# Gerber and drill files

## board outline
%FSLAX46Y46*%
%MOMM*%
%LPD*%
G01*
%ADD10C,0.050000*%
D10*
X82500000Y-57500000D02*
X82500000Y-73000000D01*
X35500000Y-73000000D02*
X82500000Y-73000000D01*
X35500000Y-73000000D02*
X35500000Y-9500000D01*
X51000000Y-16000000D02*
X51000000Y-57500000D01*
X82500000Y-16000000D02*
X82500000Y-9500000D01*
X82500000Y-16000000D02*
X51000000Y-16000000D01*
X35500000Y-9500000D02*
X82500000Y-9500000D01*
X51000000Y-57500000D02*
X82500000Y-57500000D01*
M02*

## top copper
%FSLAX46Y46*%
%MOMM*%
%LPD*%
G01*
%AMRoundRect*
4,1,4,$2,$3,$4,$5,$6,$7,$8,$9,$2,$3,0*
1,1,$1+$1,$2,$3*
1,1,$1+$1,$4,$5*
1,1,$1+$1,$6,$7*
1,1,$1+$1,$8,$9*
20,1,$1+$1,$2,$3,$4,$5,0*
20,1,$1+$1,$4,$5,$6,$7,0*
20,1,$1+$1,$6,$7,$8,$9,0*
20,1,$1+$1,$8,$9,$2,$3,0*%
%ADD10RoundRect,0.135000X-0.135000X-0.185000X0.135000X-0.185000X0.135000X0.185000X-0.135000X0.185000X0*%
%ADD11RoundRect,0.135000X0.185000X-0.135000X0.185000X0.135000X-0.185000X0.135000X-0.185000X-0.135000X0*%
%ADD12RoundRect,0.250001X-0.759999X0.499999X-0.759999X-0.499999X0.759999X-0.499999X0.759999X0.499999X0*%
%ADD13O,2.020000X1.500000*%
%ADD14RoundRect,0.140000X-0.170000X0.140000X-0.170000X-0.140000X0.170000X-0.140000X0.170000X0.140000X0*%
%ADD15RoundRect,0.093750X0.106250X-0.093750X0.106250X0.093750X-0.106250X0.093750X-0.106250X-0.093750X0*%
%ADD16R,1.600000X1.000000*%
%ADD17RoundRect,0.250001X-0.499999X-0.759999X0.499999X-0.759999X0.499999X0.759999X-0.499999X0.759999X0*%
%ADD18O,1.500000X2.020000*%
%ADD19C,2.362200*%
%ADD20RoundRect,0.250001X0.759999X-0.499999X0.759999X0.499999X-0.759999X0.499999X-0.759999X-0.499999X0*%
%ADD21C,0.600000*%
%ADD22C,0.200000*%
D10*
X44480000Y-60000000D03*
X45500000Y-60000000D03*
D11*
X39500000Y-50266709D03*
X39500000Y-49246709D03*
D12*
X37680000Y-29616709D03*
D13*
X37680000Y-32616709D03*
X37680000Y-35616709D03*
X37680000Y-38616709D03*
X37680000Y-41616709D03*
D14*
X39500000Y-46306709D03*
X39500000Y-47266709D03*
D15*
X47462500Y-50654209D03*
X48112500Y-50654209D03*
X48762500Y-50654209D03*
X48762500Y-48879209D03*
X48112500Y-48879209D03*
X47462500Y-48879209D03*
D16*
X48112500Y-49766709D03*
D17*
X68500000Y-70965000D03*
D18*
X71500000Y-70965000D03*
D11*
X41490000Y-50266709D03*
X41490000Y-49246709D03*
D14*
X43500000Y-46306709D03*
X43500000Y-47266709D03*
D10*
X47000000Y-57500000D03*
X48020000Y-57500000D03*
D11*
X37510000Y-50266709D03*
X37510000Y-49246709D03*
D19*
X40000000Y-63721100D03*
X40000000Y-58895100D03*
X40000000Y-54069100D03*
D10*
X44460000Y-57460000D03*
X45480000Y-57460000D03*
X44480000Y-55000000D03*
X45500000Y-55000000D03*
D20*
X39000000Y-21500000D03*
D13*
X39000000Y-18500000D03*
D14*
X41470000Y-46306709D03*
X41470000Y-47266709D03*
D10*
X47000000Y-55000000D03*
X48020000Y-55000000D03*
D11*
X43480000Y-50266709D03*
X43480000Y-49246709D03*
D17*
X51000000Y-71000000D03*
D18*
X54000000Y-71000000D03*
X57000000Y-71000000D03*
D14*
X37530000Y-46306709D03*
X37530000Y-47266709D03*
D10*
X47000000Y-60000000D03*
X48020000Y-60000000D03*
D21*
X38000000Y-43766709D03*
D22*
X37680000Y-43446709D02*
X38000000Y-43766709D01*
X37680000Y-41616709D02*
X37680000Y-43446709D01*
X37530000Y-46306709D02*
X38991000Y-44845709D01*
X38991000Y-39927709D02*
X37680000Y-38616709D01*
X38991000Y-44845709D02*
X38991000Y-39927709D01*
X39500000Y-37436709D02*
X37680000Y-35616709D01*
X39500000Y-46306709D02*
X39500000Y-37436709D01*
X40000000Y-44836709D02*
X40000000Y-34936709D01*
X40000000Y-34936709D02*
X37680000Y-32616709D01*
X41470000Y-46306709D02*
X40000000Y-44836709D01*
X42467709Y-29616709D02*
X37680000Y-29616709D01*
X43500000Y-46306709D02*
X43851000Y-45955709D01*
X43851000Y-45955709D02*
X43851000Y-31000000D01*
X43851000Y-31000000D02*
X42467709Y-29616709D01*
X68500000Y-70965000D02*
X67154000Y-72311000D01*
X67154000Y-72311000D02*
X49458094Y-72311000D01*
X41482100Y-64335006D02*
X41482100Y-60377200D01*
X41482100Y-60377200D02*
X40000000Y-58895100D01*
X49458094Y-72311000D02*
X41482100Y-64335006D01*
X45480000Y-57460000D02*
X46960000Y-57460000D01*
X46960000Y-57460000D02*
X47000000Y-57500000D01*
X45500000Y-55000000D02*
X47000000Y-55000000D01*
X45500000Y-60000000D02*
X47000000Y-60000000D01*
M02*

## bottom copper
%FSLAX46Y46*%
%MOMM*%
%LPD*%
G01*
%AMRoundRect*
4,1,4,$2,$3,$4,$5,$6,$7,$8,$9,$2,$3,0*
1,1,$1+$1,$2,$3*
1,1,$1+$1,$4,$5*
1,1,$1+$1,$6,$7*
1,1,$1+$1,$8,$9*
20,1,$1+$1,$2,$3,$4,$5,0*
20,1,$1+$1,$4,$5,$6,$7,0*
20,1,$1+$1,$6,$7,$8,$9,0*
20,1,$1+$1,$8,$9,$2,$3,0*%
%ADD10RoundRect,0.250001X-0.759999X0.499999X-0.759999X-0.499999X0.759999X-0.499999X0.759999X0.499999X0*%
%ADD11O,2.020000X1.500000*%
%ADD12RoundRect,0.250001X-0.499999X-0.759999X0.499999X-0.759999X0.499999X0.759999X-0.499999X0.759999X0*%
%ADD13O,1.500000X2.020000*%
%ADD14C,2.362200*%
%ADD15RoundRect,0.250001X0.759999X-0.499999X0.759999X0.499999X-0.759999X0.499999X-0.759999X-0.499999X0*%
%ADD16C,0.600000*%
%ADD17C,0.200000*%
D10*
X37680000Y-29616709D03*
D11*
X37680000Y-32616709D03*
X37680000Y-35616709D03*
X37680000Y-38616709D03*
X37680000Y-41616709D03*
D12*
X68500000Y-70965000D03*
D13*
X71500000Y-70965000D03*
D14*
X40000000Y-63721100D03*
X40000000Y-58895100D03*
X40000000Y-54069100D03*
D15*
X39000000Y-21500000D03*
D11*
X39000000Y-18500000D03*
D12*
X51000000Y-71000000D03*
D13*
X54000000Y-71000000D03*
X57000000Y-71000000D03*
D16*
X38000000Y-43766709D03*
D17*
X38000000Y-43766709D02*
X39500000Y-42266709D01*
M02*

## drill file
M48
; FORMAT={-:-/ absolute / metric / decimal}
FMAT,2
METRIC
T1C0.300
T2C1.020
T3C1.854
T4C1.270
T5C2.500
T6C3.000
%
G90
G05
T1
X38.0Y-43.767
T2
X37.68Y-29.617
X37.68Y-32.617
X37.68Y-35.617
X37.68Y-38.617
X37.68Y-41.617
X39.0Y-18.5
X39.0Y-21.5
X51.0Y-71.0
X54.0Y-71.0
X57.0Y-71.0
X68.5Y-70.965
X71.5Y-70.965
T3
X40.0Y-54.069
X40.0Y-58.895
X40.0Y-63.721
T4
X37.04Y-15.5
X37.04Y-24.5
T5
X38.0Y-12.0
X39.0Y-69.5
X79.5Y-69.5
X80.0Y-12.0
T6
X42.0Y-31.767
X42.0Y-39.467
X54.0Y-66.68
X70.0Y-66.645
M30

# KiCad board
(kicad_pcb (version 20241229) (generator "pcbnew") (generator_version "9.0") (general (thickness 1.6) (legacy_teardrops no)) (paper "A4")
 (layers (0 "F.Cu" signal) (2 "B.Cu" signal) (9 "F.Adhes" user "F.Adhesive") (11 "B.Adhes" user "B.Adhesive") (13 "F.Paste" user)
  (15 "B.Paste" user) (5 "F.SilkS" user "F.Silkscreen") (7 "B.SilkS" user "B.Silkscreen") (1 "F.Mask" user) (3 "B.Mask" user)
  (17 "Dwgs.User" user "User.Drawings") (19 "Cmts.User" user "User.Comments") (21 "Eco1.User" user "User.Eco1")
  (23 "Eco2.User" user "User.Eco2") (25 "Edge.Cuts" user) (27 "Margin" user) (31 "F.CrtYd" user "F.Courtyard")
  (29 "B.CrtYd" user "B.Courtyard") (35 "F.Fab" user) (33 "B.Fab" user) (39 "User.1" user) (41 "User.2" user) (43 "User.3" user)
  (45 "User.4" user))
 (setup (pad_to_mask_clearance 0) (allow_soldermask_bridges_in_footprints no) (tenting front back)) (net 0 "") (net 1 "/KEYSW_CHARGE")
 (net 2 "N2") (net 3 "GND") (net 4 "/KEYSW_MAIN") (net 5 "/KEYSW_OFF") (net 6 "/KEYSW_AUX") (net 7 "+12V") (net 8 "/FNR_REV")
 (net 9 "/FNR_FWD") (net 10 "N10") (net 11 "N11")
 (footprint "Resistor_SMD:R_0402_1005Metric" (layer "F.Cu") (at 44.99 60)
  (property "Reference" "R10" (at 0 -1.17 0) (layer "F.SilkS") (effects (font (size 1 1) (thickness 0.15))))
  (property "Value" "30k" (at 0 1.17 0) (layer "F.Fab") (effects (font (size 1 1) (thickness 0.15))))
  (pad "1" smd roundrect (at -0.51 0) (size 0.54 0.64) (layers "F.Cu" "F.Mask" "F.Paste") (roundrect_rratio 0.25) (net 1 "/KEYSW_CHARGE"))
  (pad "2" smd roundrect (at 0.51 0) (size 0.54 0.64) (layers "F.Cu" "F.Mask" "F.Paste") (roundrect_rratio 0.25) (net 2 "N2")))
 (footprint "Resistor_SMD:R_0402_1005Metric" (layer "F.Cu") (at 39.5 49.756709 90)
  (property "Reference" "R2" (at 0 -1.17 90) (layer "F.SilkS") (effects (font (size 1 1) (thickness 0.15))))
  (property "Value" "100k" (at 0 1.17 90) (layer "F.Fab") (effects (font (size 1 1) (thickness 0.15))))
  (pad "1" smd roundrect (at -0.51 0 90) (size 0.54 0.64) (layers "F.Cu" "F.Mask" "F.Paste") (roundrect_rratio 0.25) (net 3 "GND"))
  (pad "2" smd roundrect (at 0.51 0 90) (size 0.54 0.64) (layers "F.Cu" "F.Mask" "F.Paste") (roundrect_rratio 0.25) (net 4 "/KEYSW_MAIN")))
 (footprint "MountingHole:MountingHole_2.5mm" (layer "F.Cu") (at 79.5 69.5)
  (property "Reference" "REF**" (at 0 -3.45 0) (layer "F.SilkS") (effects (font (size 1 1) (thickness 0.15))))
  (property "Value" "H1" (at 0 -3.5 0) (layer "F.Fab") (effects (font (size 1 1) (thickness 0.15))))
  (pad "" np_thru_hole circle (at 0 0) (size 2.5 2.5) (drill 2.5) (layers "*.Cu" "*.Mask")))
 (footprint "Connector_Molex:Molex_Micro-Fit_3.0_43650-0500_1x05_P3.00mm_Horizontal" (layer "F.Cu") (at 37.68 29.616709 -90)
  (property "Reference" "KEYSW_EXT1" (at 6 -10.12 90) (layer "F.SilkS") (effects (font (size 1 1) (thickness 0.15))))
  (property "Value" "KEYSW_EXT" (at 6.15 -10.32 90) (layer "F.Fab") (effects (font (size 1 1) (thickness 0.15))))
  (pad "" np_thru_hole circle (at 2.15 -4.32 270) (size 3 3) (drill 3) (layers "*.Cu" "*.Mask"))
  (pad "" np_thru_hole circle (at 9.85 -4.32 270) (size 3 3) (drill 3) (layers "*.Cu" "*.Mask"))
  (pad "1" thru_hole roundrect (at 0 0 270) (size 1.5 2.02) (drill 1.02) (layers "*.Cu" "*.Mask") (remove_unused_layers no)
   (roundrect_rratio 0.166667) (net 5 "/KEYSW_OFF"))
  (pad "2" thru_hole oval (at 3 0 270) (size 1.5 2.02) (drill 1.02) (layers "*.Cu" "*.Mask") (remove_unused_layers no) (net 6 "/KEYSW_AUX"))
  (pad "3" thru_hole oval (at 6 0 270) (size 1.5 2.02) (drill 1.02) (layers "*.Cu" "*.Mask") (remove_unused_layers no) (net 4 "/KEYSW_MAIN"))
  (pad "4" thru_hole oval (at 9 0 270) (size 1.5 2.02) (drill 1.02) (layers "*.Cu" "*.Mask") (remove_unused_layers no)
   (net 1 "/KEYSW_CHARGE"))
  (pad "5" thru_hole oval (at 12 0 270) (size 1.5 2.02) (drill 1.02) (layers "*.Cu" "*.Mask") (remove_unused_layers no) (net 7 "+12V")))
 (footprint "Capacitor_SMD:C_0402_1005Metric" (layer "F.Cu") (at 39.5 46.786709 -90)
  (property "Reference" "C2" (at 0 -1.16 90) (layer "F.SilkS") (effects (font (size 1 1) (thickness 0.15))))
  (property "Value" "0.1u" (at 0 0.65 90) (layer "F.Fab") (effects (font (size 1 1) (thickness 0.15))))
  (pad "1" smd roundrect (at -0.48 0 270) (size 0.56 0.62) (layers "F.Cu" "F.Mask" "F.Paste") (roundrect_rratio 0.25) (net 4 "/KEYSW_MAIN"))
  (pad "2" smd roundrect (at 0.48 0 270) (size 0.56 0.62) (layers "F.Cu" "F.Mask" "F.Paste") (roundrect_rratio 0.25) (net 3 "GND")))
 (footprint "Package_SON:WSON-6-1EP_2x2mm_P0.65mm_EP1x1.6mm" (layer "F.Cu") (at 48.1125 49.766709 90)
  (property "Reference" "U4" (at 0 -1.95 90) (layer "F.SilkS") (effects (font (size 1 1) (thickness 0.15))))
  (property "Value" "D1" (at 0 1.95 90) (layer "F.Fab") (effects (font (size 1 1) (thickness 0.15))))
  (pad "" smd roundrect (at 0 -0.4 90) (size 0.81 0.64) (layers "F.Paste") (roundrect_rratio 0.25))
  (pad "" smd roundrect (at 0 0.4 90) (size 0.81 0.64) (layers "F.Paste") (roundrect_rratio 0.25))
  (pad "1" smd roundrect (at -0.8875 -0.65 90) (size 0.375 0.4) (layers "F.Cu" "F.Mask" "F.Paste") (roundrect_rratio 0.25) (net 2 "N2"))
  (pad "2" smd roundrect (at -0.8875 0 90) (size 0.375 0.4) (layers "F.Cu" "F.Mask" "F.Paste") (roundrect_rratio 0.25) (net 2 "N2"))
  (pad "3" smd roundrect (at -0.8875 0.65 90) (size 0.375 0.4) (layers "F.Cu" "F.Mask" "F.Paste") (roundrect_rratio 0.25) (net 2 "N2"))
  (pad "4" smd roundrect (at 0.8875 0.65 90) (size 0.375 0.4) (layers "F.Cu" "F.Mask" "F.Paste") (roundrect_rratio 0.25) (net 3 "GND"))
  (pad "5" smd roundrect (at 0.8875 0 90) (size 0.375 0.4) (layers "F.Cu" "F.Mask" "F.Paste") (roundrect_rratio 0.25) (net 3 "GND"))
  (pad "6" smd roundrect (at 0.8875 -0.65 90) (size 0.375 0.4) (layers "F.Cu" "F.Mask" "F.Paste") (roundrect_rratio 0.25) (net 3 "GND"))
  (pad "7" smd rect (at 0 0 90) (size 1 1.6) (layers "F.Cu" "F.Mask") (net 2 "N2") (zone_connect 2)))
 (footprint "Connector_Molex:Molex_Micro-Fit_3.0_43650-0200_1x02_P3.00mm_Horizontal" (layer "F.Cu") (at 68.5 70.965)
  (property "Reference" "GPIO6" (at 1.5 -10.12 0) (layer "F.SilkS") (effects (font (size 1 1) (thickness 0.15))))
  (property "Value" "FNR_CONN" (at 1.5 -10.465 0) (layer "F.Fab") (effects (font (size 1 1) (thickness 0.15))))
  (pad "" np_thru_hole circle (at 1.5 -4.32) (size 3 3) (drill 3) (layers "*.Cu" "*.Mask"))
  (pad "1" thru_hole roundrect (at 0 0) (size 1.5 2.02) (drill 1.02) (layers "*.Cu" "*.Mask") (remove_unused_layers no)
   (roundrect_rratio 0.166667) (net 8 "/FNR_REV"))
  (pad "2" thru_hole oval (at 3 0) (size 1.5 2.02) (drill 1.02) (layers "*.Cu" "*.Mask") (remove_unused_layers no) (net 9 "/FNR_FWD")))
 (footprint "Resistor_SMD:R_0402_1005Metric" (layer "F.Cu") (at 41.49 49.756709 90)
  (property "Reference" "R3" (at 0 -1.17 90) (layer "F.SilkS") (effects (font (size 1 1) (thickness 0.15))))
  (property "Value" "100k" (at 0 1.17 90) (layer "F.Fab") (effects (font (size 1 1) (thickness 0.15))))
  (pad "1" smd roundrect (at -0.51 0 90) (size 0.54 0.64) (layers "F.Cu" "F.Mask" "F.Paste") (roundrect_rratio 0.25) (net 3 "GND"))
  (pad "2" smd roundrect (at 0.51 0 90) (size 0.54 0.64) (layers "F.Cu" "F.Mask" "F.Paste") (roundrect_rratio 0.25) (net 6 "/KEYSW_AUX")))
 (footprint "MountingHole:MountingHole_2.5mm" (layer "F.Cu") (at 39 69.5)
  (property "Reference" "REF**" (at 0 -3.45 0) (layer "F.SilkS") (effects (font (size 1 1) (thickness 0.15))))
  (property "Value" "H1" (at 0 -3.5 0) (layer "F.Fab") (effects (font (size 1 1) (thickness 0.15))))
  (pad "" np_thru_hole circle (at 0 0) (size 2.5 2.5) (drill 2.5) (layers "*.Cu" "*.Mask")))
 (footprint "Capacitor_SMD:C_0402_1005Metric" (layer "F.Cu") (at 43.5 46.786709 -90)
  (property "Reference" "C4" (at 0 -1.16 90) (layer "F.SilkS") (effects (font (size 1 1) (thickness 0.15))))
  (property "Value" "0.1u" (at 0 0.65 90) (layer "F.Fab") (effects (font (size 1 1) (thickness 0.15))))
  (pad "1" smd roundrect (at -0.48 0 270) (size 0.56 0.62) (layers "F.Cu" "F.Mask" "F.Paste") (roundrect_rratio 0.25) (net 5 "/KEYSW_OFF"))
  (pad "2" smd roundrect (at 0.48 0 270) (size 0.56 0.62) (layers "F.Cu" "F.Mask" "F.Paste") (roundrect_rratio 0.25) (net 3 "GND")))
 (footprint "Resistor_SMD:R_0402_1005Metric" (layer "F.Cu") (at 47.51 57.5)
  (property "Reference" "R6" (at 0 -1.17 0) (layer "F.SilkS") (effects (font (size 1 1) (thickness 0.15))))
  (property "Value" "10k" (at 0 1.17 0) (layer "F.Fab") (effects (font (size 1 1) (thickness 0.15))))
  (pad "1" smd roundrect (at -0.51 0) (size 0.54 0.64) (layers "F.Cu" "F.Mask" "F.Paste") (roundrect_rratio 0.25) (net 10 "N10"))
  (pad "2" smd roundrect (at 0.51 0) (size 0.54 0.64) (layers "F.Cu" "F.Mask" "F.Paste") (roundrect_rratio 0.25) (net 3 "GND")))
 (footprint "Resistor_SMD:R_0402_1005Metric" (layer "F.Cu") (at 37.51 49.756709 90)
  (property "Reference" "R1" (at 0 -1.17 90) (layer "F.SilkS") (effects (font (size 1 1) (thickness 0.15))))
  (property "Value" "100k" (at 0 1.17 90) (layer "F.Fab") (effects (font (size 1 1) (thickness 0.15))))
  (pad "1" smd roundrect (at -0.51 0 90) (size 0.54 0.64) (layers "F.Cu" "F.Mask" "F.Paste") (roundrect_rratio 0.25) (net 3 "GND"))
  (pad "2" smd roundrect (at 0.51 0 90) (size 0.54 0.64) (layers "F.Cu" "F.Mask" "F.Paste") (roundrect_rratio 0.25) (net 1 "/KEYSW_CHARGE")))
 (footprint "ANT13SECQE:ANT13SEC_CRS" (layer "F.Cu") (at 40 63.7211 90)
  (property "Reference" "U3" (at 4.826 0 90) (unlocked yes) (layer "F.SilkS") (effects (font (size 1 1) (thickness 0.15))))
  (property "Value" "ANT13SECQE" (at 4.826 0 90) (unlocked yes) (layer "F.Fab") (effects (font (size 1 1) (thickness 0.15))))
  (pad "1" thru_hole circle (at 0 0 90) (size 2.3622 2.3622) (drill 1.8542) (layers "*.Cu" "*.Mask") (remove_unused_layers no) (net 3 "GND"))
  (pad "2" thru_hole circle (at 4.826 0 90) (size 2.3622 2.3622) (drill 1.8542) (layers "*.Cu" "*.Mask") (remove_unused_layers no)
   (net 8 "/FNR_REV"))
  (pad "3" thru_hole circle (at 9.652 0 90) (size 2.3622 2.3622) (drill 1.8542) (layers "*.Cu" "*.Mask") (remove_unused_layers no)
   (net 9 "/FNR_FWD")))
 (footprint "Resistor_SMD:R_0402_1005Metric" (layer "F.Cu") (at 44.97 57.46)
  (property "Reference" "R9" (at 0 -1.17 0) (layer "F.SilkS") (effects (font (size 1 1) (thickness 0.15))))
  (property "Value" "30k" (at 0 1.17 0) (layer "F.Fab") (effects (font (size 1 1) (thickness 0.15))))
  (pad "1" smd roundrect (at -0.51 0) (size 0.54 0.64) (layers "F.Cu" "F.Mask" "F.Paste") (roundrect_rratio 0.25) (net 4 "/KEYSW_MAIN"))
  (pad "2" smd roundrect (at 0.51 0) (size 0.54 0.64) (layers "F.Cu" "F.Mask" "F.Paste") (roundrect_rratio 0.25) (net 10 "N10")))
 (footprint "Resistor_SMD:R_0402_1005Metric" (layer "F.Cu") (at 44.99 55)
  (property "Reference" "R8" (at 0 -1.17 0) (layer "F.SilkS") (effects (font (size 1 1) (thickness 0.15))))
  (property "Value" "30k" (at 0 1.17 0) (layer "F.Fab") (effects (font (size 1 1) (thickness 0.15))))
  (pad "1" smd roundrect (at -0.51 0) (size 0.54 0.64) (layers "F.Cu" "F.Mask" "F.Paste") (roundrect_rratio 0.25) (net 6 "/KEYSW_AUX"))
  (pad "2" smd roundrect (at 0.51 0) (size 0.54 0.64) (layers "F.Cu" "F.Mask" "F.Paste") (roundrect_rratio 0.25) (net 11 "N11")))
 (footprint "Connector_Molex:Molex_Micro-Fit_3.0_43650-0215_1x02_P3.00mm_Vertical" (layer "F.Cu") (at 39 21.5 90)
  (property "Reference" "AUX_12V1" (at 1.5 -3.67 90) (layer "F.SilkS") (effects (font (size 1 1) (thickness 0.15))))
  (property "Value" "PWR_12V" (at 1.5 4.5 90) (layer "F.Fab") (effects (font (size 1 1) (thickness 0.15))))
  (pad "" np_thru_hole circle (at -3 -1.96 90) (size 1.27 1.27) (drill 1.27) (layers "*.Cu" "*.Mask"))
  (pad "" np_thru_hole circle (at 6 -1.96 90) (size 1.27 1.27) (drill 1.27) (layers "*.Cu" "*.Mask"))
  (pad "1" thru_hole roundrect (at 0 0 90) (size 1.5 2.02) (drill 1.02) (layers "*.Cu" "*.Mask") (remove_unused_layers no)
   (roundrect_rratio 0.166667) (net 7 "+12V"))
  (pad "2" thru_hole oval (at 3 0 90) (size 1.5 2.02) (drill 1.02) (layers "*.Cu" "*.Mask") (remove_unused_layers no) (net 3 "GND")))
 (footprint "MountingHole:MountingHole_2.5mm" (layer "F.Cu") (at 80 12)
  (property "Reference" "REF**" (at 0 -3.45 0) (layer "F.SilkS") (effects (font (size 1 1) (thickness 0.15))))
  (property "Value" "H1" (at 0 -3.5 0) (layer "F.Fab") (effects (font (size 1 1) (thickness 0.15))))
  (pad "" np_thru_hole circle (at 0 0) (size 2.5 2.5) (drill 2.5) (layers "*.Cu" "*.Mask")))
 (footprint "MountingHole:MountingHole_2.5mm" (layer "F.Cu") (at 38 12)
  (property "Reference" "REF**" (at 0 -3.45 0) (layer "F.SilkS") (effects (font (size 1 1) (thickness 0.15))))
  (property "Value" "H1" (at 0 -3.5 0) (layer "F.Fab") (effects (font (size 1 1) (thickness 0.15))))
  (pad "" np_thru_hole circle (at 0 0) (size 2.5 2.5) (drill 2.5) (layers "*.Cu" "*.Mask")))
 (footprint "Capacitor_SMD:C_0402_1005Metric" (layer "F.Cu") (at 41.47 46.786709 -90)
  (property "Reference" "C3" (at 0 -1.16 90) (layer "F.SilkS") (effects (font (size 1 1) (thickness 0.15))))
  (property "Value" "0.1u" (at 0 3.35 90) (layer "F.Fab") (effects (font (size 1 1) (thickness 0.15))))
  (pad "1" smd roundrect (at -0.48 0 270) (size 0.56 0.62) (layers "F.Cu" "F.Mask" "F.Paste") (roundrect_rratio 0.25) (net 6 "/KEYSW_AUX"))
  (pad "2" smd roundrect (at 0.48 0 270) (size 0.56 0.62) (layers "F.Cu" "F.Mask" "F.Paste") (roundrect_rratio 0.25) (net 3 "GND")))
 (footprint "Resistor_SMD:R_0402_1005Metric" (layer "F.Cu") (at 47.51 55)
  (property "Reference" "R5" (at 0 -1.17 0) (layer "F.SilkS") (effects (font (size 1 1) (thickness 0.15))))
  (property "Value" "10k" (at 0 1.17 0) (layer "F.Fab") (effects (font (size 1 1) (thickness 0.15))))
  (pad "1" smd roundrect (at -0.51 0) (size 0.54 0.64) (layers "F.Cu" "F.Mask" "F.Paste") (roundrect_rratio 0.25) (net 11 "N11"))
  (pad "2" smd roundrect (at 0.51 0) (size 0.54 0.64) (layers "F.Cu" "F.Mask" "F.Paste") (roundrect_rratio 0.25) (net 3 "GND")))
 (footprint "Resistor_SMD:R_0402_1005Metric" (layer "F.Cu") (at 43.48 49.756709 90)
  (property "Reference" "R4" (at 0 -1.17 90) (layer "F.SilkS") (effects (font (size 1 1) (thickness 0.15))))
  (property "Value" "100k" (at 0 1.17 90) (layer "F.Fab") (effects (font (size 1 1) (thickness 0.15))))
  (pad "1" smd roundrect (at -0.51 0 90) (size 0.54 0.64) (layers "F.Cu" "F.Mask" "F.Paste") (roundrect_rratio 0.25) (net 3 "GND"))
  (pad "2" smd roundrect (at 0.51 0 90) (size 0.54 0.64) (layers "F.Cu" "F.Mask" "F.Paste") (roundrect_rratio 0.25) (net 5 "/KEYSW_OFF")))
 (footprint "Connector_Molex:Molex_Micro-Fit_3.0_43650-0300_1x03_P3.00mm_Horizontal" (layer "F.Cu") (at 51 71)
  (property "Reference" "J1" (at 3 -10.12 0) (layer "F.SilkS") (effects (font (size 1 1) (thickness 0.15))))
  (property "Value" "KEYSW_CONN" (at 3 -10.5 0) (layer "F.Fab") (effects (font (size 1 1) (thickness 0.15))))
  (pad "" np_thru_hole circle (at 3 -4.32) (size 3 3) (drill 3) (layers "*.Cu" "*.Mask"))
  (pad "1" thru_hole roundrect (at 0 0) (size 1.5 2.02) (drill 1.02) (layers "*.Cu" "*.Mask") (remove_unused_layers no)
   (roundrect_rratio 0.166667) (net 11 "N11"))
  (pad "2" thru_hole oval (at 3 0) (size 1.5 2.02) (drill 1.02) (layers "*.Cu" "*.Mask") (remove_unused_layers no) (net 10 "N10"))
  (pad "3" thru_hole oval (at 6 0) (size 1.5 2.02) (drill 1.02) (layers "*.Cu" "*.Mask") (remove_unused_layers no) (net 2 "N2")))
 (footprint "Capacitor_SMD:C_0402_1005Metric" (layer "F.Cu") (at 37.53 46.786709 -90)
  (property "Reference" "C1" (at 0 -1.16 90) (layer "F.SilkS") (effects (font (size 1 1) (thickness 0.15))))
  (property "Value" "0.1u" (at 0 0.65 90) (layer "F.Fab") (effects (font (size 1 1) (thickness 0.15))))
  (pad "1" smd roundrect (at -0.48 0 270) (size 0.56 0.62) (layers "F.Cu" "F.Mask" "F.Paste") (roundrect_rratio 0.25)
   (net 1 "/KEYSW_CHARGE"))
  (pad "2" smd roundrect (at 0.48 0 270) (size 0.56 0.62) (layers "F.Cu" "F.Mask" "F.Paste") (roundrect_rratio 0.25) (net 3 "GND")))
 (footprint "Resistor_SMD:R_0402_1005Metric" (layer "F.Cu") (at 47.51 60)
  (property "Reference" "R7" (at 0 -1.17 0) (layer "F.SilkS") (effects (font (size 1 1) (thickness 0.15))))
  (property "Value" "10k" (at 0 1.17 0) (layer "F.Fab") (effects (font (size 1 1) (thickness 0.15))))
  (pad "1" smd roundrect (at -0.51 0) (size 0.54 0.64) (layers "F.Cu" "F.Mask" "F.Paste") (roundrect_rratio 0.25) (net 2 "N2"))
  (pad "2" smd roundrect (at 0.51 0) (size 0.54 0.64) (layers "F.Cu" "F.Mask" "F.Paste") (roundrect_rratio 0.25) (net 3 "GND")))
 (gr_line (start 82.5 57.5) (end 82.5 73) (stroke (width 0.05) (type default)) (layer "Edge.Cuts"))
 (gr_line (start 35.5 73) (end 82.5 73) (stroke (width 0.05) (type default)) (layer "Edge.Cuts"))
 (gr_line (start 35.5 73) (end 35.5 9.5) (stroke (width 0.05) (type default)) (layer "Edge.Cuts"))
 (gr_line (start 51 16) (end 51 57.5) (stroke (width 0.05) (type default)) (layer "Edge.Cuts"))
 (gr_line (start 82.5 16) (end 82.5 9.5) (stroke (width 0.05) (type default)) (layer "Edge.Cuts"))
 (gr_line (start 82.5 16) (end 51 16) (stroke (width 0.05) (type default)) (layer "Edge.Cuts"))
 (gr_line (start 35.5 9.5) (end 82.5 9.5) (stroke (width 0.05) (type default)) (layer "Edge.Cuts"))
 (gr_line (start 51 57.5) (end 82.5 57.5) (stroke (width 0.05) (type default)) (layer "Edge.Cuts"))
 (segment (start 37.68 43.446709) (end 38 43.766709) (width 0.2) (layer "F.Cu") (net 7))
 (segment (start 37.68 41.616709) (end 37.68 43.446709) (width 0.2) (layer "F.Cu") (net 7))
 (via (at 38 43.766709) (size 0.6) (drill 0.3) (layers "F.Cu" "B.Cu") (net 7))
 (segment (start 38 43.766709) (end 39.5 42.266709) (width 0.2) (layer "B.Cu") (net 7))
 (segment (start 37.53 46.306709) (end 38.991 44.845709) (width 0.2) (layer "F.Cu") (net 1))
 (segment (start 38.991 39.927709) (end 37.68 38.616709) (width 0.2) (layer "F.Cu") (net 1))
 (segment (start 38.991 44.845709) (end 38.991 39.927709) (width 0.2) (layer "F.Cu") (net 1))
 (segment (start 39.5 37.436709) (end 37.68 35.616709) (width 0.2) (layer "F.Cu") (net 4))
 (segment (start 39.5 46.306709) (end 39.5 37.436709) (width 0.2) (layer "F.Cu") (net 4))
 (segment (start 40 44.836709) (end 40 34.936709) (width 0.2) (layer "F.Cu") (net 6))
 (segment (start 40 34.936709) (end 37.68 32.616709) (width 0.2) (layer "F.Cu") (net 6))
 (segment (start 41.47 46.306709) (end 40 44.836709) (width 0.2) (layer "F.Cu") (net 6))
 (segment (start 42.467709 29.616709) (end 37.68 29.616709) (width 0.2) (layer "F.Cu") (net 5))
 (segment (start 43.5 46.306709) (end 43.851 45.955709) (width 0.2) (layer "F.Cu") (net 5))
 (segment (start 43.851 45.955709) (end 43.851 31) (width 0.2) (layer "F.Cu") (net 5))
 (segment (start 43.851 31) (end 42.467709 29.616709) (width 0.2) (layer "F.Cu") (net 5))
 (segment (start 68.5 70.965) (end 67.154 72.311) (width 0.2) (layer "F.Cu") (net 8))
 (segment (start 67.154 72.311) (end 49.458094 72.311) (width 0.2) (layer "F.Cu") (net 8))
 (segment (start 41.4821 64.335006) (end 41.4821 60.3772) (width 0.2) (layer "F.Cu") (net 8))
 (segment (start 41.4821 60.3772) (end 40 58.8951) (width 0.2) (layer "F.Cu") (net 8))
 (segment (start 49.458094 72.311) (end 41.4821 64.335006) (width 0.2) (layer "F.Cu") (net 8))
 (segment (start 45.48 57.46) (end 46.96 57.46) (width 0.2) (layer "F.Cu") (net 10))
 (segment (start 46.96 57.46) (end 47 57.5) (width 0.2) (layer "F.Cu") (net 10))
 (segment (start 45.5 55) (end 47 55) (width 0.2) (layer "F.Cu") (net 11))
 (segment (start 45.5 60) (end 47 60) (width 0.2) (layer "F.Cu") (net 2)))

